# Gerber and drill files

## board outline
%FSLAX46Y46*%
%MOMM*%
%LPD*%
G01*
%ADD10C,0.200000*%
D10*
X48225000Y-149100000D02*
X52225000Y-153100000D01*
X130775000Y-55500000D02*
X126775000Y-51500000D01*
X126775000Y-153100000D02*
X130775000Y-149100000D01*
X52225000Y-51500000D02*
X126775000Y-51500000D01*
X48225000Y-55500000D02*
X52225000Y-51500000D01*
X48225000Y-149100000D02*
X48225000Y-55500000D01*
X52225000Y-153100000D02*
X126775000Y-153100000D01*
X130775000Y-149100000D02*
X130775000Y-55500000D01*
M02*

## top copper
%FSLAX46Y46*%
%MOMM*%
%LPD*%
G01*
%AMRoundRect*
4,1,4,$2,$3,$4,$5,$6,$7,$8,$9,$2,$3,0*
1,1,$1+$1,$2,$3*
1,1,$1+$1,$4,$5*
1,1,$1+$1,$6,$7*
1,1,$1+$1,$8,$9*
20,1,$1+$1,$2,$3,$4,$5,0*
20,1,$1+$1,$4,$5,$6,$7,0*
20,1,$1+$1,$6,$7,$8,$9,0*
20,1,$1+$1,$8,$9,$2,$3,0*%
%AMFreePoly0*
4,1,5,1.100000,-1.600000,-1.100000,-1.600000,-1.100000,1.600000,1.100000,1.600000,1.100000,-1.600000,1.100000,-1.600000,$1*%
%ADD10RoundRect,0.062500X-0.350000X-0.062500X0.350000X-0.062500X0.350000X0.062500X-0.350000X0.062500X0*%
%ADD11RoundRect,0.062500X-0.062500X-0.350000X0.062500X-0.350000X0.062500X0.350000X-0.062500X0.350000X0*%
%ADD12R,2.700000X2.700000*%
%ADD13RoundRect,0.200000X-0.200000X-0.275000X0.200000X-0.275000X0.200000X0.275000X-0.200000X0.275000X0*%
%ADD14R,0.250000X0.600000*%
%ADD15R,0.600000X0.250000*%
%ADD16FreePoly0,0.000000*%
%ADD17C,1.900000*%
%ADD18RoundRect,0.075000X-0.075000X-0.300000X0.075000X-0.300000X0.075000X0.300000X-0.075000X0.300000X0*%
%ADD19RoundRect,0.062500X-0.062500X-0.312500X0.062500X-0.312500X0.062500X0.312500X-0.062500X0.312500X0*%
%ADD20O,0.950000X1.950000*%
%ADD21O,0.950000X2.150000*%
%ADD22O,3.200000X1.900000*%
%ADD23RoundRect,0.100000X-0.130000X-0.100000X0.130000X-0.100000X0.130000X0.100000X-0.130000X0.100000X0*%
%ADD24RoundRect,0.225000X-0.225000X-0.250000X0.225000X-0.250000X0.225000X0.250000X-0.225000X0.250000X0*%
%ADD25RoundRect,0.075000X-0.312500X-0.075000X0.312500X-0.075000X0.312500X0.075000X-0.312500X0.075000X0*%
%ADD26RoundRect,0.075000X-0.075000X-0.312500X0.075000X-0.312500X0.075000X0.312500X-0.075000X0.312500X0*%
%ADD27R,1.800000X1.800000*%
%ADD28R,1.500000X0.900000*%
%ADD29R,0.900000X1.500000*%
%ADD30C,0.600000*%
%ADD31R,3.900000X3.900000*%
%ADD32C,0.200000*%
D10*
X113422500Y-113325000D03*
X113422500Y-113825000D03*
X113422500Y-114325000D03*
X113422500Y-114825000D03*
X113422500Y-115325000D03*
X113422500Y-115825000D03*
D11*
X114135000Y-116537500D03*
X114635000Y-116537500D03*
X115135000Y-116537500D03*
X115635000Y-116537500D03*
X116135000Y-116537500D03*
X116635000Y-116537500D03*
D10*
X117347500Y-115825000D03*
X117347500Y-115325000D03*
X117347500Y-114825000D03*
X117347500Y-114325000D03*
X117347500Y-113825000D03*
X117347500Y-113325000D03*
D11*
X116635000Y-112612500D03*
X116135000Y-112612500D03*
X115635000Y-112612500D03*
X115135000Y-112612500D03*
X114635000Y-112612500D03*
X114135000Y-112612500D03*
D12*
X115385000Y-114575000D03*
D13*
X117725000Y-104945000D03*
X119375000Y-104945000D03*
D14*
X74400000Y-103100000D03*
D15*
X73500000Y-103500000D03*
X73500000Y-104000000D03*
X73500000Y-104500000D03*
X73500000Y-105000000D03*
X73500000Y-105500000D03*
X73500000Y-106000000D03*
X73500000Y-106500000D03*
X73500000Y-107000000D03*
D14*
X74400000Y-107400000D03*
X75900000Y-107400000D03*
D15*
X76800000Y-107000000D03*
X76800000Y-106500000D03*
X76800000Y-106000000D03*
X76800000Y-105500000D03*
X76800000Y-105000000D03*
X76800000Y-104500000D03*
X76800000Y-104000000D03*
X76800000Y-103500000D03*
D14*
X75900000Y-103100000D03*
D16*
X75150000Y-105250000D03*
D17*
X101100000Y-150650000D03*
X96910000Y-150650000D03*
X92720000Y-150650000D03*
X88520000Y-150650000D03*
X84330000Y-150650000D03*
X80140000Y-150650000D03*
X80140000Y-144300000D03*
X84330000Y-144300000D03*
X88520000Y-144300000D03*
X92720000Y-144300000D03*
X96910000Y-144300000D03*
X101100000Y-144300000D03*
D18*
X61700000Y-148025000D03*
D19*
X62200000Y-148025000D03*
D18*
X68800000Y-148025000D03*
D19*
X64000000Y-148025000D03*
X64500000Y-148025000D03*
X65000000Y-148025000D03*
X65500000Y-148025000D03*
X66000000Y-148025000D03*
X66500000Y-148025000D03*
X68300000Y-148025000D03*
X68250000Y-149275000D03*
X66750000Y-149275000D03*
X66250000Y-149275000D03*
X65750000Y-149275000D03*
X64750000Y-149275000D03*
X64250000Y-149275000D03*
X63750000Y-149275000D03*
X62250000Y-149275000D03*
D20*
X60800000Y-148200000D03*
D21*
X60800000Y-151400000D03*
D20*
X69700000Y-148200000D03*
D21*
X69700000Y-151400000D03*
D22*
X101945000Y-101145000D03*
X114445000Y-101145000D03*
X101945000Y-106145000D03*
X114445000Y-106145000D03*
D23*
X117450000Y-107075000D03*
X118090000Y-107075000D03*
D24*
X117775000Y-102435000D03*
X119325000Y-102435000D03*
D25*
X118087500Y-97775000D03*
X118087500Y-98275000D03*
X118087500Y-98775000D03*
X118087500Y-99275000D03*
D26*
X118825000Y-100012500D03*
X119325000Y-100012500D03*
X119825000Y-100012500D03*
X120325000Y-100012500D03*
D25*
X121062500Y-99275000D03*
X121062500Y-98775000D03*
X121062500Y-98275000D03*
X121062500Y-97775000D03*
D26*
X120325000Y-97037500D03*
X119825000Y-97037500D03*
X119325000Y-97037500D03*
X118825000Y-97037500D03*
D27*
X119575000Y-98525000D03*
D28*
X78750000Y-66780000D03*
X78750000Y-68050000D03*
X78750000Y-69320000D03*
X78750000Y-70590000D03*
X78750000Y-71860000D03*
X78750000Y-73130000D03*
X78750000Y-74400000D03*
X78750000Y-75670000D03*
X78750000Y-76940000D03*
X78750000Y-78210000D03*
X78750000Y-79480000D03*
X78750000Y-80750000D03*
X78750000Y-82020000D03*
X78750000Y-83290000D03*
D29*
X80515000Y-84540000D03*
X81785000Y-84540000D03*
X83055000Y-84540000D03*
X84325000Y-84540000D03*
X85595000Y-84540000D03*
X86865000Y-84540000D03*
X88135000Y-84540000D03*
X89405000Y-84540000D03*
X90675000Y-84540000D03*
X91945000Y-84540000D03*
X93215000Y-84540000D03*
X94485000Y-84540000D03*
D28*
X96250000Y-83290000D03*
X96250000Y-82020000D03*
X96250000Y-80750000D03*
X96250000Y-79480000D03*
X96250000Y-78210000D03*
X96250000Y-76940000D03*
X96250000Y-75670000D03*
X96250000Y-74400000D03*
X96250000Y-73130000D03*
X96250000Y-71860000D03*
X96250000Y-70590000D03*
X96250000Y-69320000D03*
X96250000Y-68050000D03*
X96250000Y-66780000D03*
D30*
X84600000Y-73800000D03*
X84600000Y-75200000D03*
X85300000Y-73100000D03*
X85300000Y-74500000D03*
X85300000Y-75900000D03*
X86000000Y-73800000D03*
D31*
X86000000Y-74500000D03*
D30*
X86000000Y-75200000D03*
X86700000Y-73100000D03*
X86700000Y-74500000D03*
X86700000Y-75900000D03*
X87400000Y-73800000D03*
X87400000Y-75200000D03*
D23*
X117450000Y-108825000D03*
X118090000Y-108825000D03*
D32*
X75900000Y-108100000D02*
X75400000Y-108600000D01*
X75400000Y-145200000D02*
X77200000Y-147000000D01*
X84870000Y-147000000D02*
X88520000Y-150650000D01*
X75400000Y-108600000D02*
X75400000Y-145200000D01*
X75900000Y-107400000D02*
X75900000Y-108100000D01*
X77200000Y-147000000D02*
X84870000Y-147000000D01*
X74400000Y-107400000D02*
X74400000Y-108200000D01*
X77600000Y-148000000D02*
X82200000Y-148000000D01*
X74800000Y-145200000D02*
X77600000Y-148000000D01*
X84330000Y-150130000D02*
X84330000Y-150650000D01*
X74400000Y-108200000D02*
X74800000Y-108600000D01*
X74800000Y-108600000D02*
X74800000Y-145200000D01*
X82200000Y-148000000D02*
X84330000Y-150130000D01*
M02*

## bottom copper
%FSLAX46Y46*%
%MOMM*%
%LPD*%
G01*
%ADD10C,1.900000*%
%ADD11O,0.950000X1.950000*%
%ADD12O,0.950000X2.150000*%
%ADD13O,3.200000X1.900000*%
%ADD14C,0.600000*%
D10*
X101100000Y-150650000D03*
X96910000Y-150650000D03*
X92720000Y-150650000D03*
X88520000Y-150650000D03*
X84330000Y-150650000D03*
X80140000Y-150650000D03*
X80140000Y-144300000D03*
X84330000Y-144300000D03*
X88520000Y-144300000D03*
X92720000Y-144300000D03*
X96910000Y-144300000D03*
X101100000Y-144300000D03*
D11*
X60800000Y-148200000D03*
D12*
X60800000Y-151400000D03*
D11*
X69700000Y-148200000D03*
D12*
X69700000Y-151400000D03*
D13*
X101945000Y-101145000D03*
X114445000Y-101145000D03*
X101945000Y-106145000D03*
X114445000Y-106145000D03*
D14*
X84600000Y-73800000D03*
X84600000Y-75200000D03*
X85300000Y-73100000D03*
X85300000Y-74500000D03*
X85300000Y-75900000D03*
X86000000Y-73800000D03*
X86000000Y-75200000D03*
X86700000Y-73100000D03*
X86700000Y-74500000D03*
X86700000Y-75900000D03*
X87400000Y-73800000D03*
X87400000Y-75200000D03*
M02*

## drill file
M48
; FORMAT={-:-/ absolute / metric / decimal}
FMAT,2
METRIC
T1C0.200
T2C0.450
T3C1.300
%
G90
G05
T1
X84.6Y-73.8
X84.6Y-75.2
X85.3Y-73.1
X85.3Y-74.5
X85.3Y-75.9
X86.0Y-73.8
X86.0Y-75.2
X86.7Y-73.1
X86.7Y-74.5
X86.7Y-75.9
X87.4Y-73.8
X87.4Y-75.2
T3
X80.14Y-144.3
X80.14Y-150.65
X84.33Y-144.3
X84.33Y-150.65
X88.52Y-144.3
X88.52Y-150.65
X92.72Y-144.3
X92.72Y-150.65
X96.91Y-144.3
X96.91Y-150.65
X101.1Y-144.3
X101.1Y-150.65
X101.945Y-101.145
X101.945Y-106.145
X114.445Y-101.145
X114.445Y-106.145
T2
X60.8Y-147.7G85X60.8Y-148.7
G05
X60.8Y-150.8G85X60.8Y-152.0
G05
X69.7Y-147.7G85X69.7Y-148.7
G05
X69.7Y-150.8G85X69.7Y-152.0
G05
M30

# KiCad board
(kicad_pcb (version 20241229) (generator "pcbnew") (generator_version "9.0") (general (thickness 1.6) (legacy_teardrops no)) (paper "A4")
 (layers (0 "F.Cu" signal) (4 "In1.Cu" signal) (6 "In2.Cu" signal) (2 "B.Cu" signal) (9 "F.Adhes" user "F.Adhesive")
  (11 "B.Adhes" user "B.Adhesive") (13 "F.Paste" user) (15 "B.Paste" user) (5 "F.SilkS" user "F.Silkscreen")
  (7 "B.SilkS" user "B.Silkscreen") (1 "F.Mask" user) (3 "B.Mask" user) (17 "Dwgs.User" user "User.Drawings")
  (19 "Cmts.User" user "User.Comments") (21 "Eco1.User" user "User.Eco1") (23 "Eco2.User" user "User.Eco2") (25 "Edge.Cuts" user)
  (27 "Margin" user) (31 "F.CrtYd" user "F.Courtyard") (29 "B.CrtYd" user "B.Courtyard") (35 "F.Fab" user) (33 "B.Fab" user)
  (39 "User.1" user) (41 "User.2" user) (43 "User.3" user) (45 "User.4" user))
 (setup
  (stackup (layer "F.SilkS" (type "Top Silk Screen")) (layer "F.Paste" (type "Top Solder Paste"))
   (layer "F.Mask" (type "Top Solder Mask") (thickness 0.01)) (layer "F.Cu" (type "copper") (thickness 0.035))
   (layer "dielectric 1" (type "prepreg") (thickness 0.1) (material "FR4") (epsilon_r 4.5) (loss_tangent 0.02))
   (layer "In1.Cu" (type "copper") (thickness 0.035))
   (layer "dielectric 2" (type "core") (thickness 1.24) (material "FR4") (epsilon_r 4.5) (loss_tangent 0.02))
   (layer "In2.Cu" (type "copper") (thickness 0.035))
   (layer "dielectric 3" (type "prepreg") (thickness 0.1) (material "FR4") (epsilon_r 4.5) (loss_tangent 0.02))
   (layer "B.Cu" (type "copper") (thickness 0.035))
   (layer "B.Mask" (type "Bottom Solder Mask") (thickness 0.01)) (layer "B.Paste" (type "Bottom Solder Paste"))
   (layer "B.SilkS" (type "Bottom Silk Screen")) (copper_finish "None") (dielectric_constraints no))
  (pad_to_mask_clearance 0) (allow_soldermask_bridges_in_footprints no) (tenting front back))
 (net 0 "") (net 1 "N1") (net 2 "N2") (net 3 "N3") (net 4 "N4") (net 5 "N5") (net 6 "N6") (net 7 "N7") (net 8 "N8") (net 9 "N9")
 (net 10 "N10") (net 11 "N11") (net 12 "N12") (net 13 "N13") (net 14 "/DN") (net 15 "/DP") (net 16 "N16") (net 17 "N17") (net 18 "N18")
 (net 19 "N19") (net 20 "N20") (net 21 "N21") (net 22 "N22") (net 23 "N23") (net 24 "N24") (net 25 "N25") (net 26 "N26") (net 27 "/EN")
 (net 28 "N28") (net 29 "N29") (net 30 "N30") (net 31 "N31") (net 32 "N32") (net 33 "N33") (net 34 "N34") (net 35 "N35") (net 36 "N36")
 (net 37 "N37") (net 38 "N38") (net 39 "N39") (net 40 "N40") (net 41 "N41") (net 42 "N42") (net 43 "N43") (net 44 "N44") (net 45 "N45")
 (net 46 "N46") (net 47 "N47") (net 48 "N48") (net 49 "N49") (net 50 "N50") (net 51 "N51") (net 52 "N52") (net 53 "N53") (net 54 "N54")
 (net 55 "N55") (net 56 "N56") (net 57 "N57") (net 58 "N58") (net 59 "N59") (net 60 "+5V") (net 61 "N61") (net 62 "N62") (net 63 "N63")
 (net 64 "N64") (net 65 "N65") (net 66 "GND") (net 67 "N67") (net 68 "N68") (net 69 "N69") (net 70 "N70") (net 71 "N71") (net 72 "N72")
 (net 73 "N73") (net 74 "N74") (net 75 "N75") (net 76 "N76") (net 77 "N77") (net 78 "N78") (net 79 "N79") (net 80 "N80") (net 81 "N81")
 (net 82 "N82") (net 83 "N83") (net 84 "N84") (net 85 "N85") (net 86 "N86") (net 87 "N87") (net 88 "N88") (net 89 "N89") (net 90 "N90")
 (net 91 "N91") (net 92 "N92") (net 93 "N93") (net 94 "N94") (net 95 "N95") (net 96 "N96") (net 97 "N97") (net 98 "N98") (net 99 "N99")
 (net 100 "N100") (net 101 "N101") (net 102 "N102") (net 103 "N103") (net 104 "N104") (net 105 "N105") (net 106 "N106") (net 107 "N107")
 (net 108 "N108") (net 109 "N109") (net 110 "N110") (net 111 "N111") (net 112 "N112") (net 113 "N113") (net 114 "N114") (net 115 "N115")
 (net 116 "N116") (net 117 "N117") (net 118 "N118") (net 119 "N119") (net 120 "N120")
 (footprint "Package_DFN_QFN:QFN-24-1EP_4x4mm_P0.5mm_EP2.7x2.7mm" (layer "F.Cu") (at 115.385 114.575)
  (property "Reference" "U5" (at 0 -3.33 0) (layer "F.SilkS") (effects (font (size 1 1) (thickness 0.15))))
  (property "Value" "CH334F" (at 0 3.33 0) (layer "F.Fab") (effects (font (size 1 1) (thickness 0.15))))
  (pad "" smd roundrect (at -0.675 -0.675) (size 1.09 1.09) (layers "F.Paste") (roundrect_rratio 0.229358))
  (pad "" smd roundrect (at -0.675 0.675) (size 1.09 1.09) (layers "F.Paste") (roundrect_rratio 0.229358))
  (pad "" smd roundrect (at 0.675 -0.675) (size 1.09 1.09) (layers "F.Paste") (roundrect_rratio 0.229358))
  (pad "" smd roundrect (at 0.675 0.675) (size 1.09 1.09) (layers "F.Paste") (roundrect_rratio 0.229358))
  (pad "1" smd roundrect (at -1.9625 -1.25) (size 0.825 0.25) (layers "F.Cu" "F.Mask" "F.Paste") (roundrect_rratio 0.25) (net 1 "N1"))
  (pad "2" smd roundrect (at -1.9625 -0.75) (size 0.825 0.25) (layers "F.Cu" "F.Mask" "F.Paste") (roundrect_rratio 0.25) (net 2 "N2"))
  (pad "3" smd roundrect (at -1.9625 -0.25) (size 0.825 0.25) (layers "F.Cu" "F.Mask" "F.Paste") (roundrect_rratio 0.25) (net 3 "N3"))
  (pad "4" smd roundrect (at -1.9625 0.25) (size 0.825 0.25) (layers "F.Cu" "F.Mask" "F.Paste") (roundrect_rratio 0.25) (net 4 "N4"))
  (pad "5" smd roundrect (at -1.9625 0.75) (size 0.825 0.25) (layers "F.Cu" "F.Mask" "F.Paste") (roundrect_rratio 0.25) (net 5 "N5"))
  (pad "6" smd roundrect (at -1.9625 1.25) (size 0.825 0.25) (layers "F.Cu" "F.Mask" "F.Paste") (roundrect_rratio 0.25) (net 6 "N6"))
  (pad "7" smd roundrect (at -1.25 1.9625) (size 0.25 0.825) (layers "F.Cu" "F.Mask" "F.Paste") (roundrect_rratio 0.25) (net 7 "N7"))
  (pad "8" smd roundrect (at -0.75 1.9625) (size 0.25 0.825) (layers "F.Cu" "F.Mask" "F.Paste") (roundrect_rratio 0.25) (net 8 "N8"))
  (pad "9" smd roundrect (at -0.25 1.9625) (size 0.25 0.825) (layers "F.Cu" "F.Mask" "F.Paste") (roundrect_rratio 0.25) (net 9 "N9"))
  (pad "10" smd roundrect (at 0.25 1.9625) (size 0.25 0.825) (layers "F.Cu" "F.Mask" "F.Paste") (roundrect_rratio 0.25) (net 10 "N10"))
  (pad "11" smd roundrect (at 0.75 1.9625) (size 0.25 0.825) (layers "F.Cu" "F.Mask" "F.Paste") (roundrect_rratio 0.25) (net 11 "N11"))
  (pad "12" smd roundrect (at 1.25 1.9625) (size 0.25 0.825) (layers "F.Cu" "F.Mask" "F.Paste") (roundrect_rratio 0.25) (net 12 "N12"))
  (pad "13" smd roundrect (at 1.9625 1.25) (size 0.825 0.25) (layers "F.Cu" "F.Mask" "F.Paste") (roundrect_rratio 0.25) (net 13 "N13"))
  (pad "14" smd roundrect (at 1.9625 0.75) (size 0.825 0.25) (layers "F.Cu" "F.Mask" "F.Paste") (roundrect_rratio 0.25) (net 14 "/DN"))
  (pad "15" smd roundrect (at 1.9625 0.25) (size 0.825 0.25) (layers "F.Cu" "F.Mask" "F.Paste") (roundrect_rratio 0.25) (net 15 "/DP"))
  (pad "16" smd roundrect (at 1.9625 -0.25) (size 0.825 0.25) (layers "F.Cu" "F.Mask" "F.Paste") (roundrect_rratio 0.25) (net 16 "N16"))
  (pad "17" smd roundrect (at 1.9625 -0.75) (size 0.825 0.25) (layers "F.Cu" "F.Mask" "F.Paste") (roundrect_rratio 0.25) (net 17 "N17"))
  (pad "18" smd roundrect (at 1.9625 -1.25) (size 0.825 0.25) (layers "F.Cu" "F.Mask" "F.Paste") (roundrect_rratio 0.25) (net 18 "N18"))
  (pad "19" smd roundrect (at 1.25 -1.9625) (size 0.25 0.825) (layers "F.Cu" "F.Mask" "F.Paste") (roundrect_rratio 0.25) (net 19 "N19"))
  (pad "20" smd roundrect (at 0.75 -1.9625) (size 0.25 0.825) (layers "F.Cu" "F.Mask" "F.Paste") (roundrect_rratio 0.25) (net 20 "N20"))
  (pad "21" smd roundrect (at 0.25 -1.9625) (size 0.25 0.825) (layers "F.Cu" "F.Mask" "F.Paste") (roundrect_rratio 0.25) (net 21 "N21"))
  (pad "22" smd roundrect (at -0.25 -1.9625) (size 0.25 0.825) (layers "F.Cu" "F.Mask" "F.Paste") (roundrect_rratio 0.25) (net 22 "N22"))
  (pad "23" smd roundrect (at -0.75 -1.9625) (size 0.25 0.825) (layers "F.Cu" "F.Mask" "F.Paste") (roundrect_rratio 0.25) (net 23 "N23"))
  (pad "24" smd roundrect (at -1.25 -1.9625) (size 0.25 0.825) (layers "F.Cu" "F.Mask" "F.Paste") (roundrect_rratio 0.25) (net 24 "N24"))
  (pad "25" smd rect (at 0 0) (size 2.7 2.7) (layers "F.Cu" "F.Mask") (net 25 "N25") (zone_connect 2)))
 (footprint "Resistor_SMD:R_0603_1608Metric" (layer "F.Cu") (at 118.55 104.945)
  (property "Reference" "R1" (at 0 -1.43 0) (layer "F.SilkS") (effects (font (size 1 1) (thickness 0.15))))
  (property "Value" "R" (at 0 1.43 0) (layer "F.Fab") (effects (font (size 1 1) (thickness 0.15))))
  (pad "1" smd roundrect (at -0.825 0) (size 0.8 0.95) (layers "F.Cu" "F.Mask" "F.Paste") (roundrect_rratio 0.25) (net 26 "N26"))
  (pad "2" smd roundrect (at 0.825 0) (size 0.8 0.95) (layers "F.Cu" "F.Mask" "F.Paste") (roundrect_rratio 0.25) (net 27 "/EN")))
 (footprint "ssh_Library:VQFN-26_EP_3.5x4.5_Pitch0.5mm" (layer "F.Cu") (at 75.15 105.25)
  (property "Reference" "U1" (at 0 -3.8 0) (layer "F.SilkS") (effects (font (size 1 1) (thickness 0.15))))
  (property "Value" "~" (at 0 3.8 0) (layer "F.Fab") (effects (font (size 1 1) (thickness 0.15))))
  (pad "" smd rect (at -0.825 -1.2) (size 0.000001 0.250001) (layers "F.Paste") (thermal_bridge_angle 45))
  (pad "" smd rect (at -0.825 -0.4) (size 0.000001 0.250001) (layers "F.Paste") (thermal_bridge_angle 45))
  (pad "" smd rect (at -0.825 0.4) (size 0.000001 0.250001) (layers "F.Paste") (thermal_bridge_angle 45))
  (pad "" smd rect (at -0.825 1.2) (size 0.000001 0.250001) (layers "F.Paste") (thermal_bridge_angle 45))
  (pad "" smd rect (at -0.275 -1.2) (size 0.000001 0.250001) (layers "F.Paste") (thermal_bridge_angle 45))
  (pad "" smd rect (at -0.275 -0.4) (size 0.000001 0.250001) (layers "F.Paste") (thermal_bridge_angle 45))
  (pad "" smd rect (at -0.275 0.4) (size 0.000001 0.250001) (layers "F.Paste") (thermal_bridge_angle 45))
  (pad "" smd rect (at -0.275 1.2) (size 0.000001 0.250001) (layers "F.Paste") (thermal_bridge_angle 45))
  (pad "" smd rect (at 0.275 -1.2) (size 0.000001 0.250001) (layers "F.Paste") (thermal_bridge_angle 45))
  (pad "" smd rect (at 0.275 -0.4) (size 0.000001 0.250001) (layers "F.Paste") (thermal_bridge_angle 45))
  (pad "" smd rect (at 0.275 0.4) (size 0.000001 0.250001) (layers "F.Paste") (thermal_bridge_angle 45))
  (pad "" smd rect (at 0.275 1.2) (size 0.000001 0.250001) (layers "F.Paste") (thermal_bridge_angle 45))
  (pad "" smd rect (at 0.825 -1.2) (size 0.000001 0.250001) (layers "F.Paste") (thermal_bridge_angle 45))
  (pad "" smd rect (at 0.825 -0.4) (size 0.000001 0.250001) (layers "F.Paste") (thermal_bridge_angle 45))
  (pad "" smd rect (at 0.825 0.4) (size 0.000001 0.250001) (layers "F.Paste") (thermal_bridge_angle 45))
  (pad "" smd rect (at 0.825 1.2) (size 0.000001 0.250001) (layers "F.Paste") (thermal_bridge_angle 45))
  (pad "1" smd rect (at -0.75 -2.15) (size 0.25 0.6) (layers "F.Cu" "F.Mask" "F.Paste") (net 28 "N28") (thermal_bridge_angle 45))
  (pad "2" smd rect (at -1.65 -1.75 90) (size 0.25 0.6) (layers "F.Cu" "F.Mask" "F.Paste") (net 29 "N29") (thermal_bridge_angle 45))
  (pad "3" smd rect (at -1.65 -1.25 90) (size 0.25 0.6) (layers "F.Cu" "F.Mask" "F.Paste") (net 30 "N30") (thermal_bridge_angle 45))
  (pad "4" smd rect (at -1.65 -0.75 90) (size 0.25 0.6) (layers "F.Cu" "F.Mask" "F.Paste") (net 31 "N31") (thermal_bridge_angle 45))
  (pad "5" smd rect (at -1.65 -0.25 90) (size 0.25 0.6) (layers "F.Cu" "F.Mask" "F.Paste") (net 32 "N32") (thermal_bridge_angle 45))
  (pad "6" smd rect (at -1.65 0.25 90) (size 0.25 0.6) (layers "F.Cu" "F.Mask" "F.Paste") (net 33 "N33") (thermal_bridge_angle 45))
  (pad "7" smd rect (at -1.65 0.75 90) (size 0.25 0.6) (layers "F.Cu" "F.Mask" "F.Paste") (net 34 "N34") (thermal_bridge_angle 45))
  (pad "8" smd rect (at -1.65 1.25 90) (size 0.25 0.6) (layers "F.Cu" "F.Mask" "F.Paste") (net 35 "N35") (thermal_bridge_angle 45))
  (pad "9" smd rect (at -1.65 1.75 90) (size 0.25 0.6) (layers "F.Cu" "F.Mask" "F.Paste") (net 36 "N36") (thermal_bridge_angle 45))
  (pad "10" smd rect (at -0.75 2.15) (size 0.25 0.6) (layers "F.Cu" "F.Mask" "F.Paste") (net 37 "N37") (thermal_bridge_angle 45))
  (pad "11" smd rect (at 0.75 2.15) (size 0.25 0.6) (layers "F.Cu" "F.Mask" "F.Paste") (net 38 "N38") (thermal_bridge_angle 45))
  (pad "12" smd rect (at 1.65 1.75 90) (size 0.25 0.6) (layers "F.Cu" "F.Mask" "F.Paste") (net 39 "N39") (thermal_bridge_angle 45))
  (pad "13" smd rect (at 1.65 1.25 90) (size 0.25 0.6) (layers "F.Cu" "F.Mask" "F.Paste") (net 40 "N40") (thermal_bridge_angle 45))
  (pad "14" smd rect (at 1.65 0.75 90) (size 0.25 0.6) (layers "F.Cu" "F.Mask" "F.Paste") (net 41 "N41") (thermal_bridge_angle 45))
  (pad "15" smd rect (at 1.65 0.25 90) (size 0.25 0.6) (layers "F.Cu" "F.Mask" "F.Paste") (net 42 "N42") (thermal_bridge_angle 45))
  (pad "16" smd rect (at 1.65 -0.25 90) (size 0.25 0.6) (layers "F.Cu" "F.Mask" "F.Paste") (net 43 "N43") (thermal_bridge_angle 45))
  (pad "17" smd rect (at 1.65 -0.75 90) (size 0.25 0.6) (layers "F.Cu" "F.Mask" "F.Paste") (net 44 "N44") (thermal_bridge_angle 45))
  (pad "18" smd rect (at 1.65 -1.25 90) (size 0.25 0.6) (layers "F.Cu" "F.Mask" "F.Paste") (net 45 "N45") (thermal_bridge_angle 45))
  (pad "19" smd rect (at 1.65 -1.75 90) (size 0.25 0.6) (layers "F.Cu" "F.Mask" "F.Paste") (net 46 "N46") (thermal_bridge_angle 45))
  (pad "20" smd rect (at 0.75 -2.15) (size 0.25 0.6) (layers "F.Cu" "F.Mask" "F.Paste") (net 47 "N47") (thermal_bridge_angle 45))
  (pad "21" smd custom (at 0 0) (size 2.2 3.2) (layers "F.Cu" "F.Mask") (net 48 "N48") (options (clearance outline) (anchor rect))
   (primitives)
   (teardrops (best_length_ratio 0.5) (max_length 1) (best_width_ratio 1) (max_width 2) (curved_edges no) (filter_ratio 0.9) (enabled yes)
    (allow_two_segments yes) (prefer_zone_connections yes))))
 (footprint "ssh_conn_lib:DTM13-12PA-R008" (layer "F.Cu") (at 90.62 153.1)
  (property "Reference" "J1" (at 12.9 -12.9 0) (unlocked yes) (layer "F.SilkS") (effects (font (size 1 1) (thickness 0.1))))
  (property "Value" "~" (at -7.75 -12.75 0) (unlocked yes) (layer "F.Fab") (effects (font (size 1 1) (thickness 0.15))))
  (pad "1" thru_hole circle (at 10.48 -2.45) (size 1.9 1.9) (drill 1.3) (layers "*.Cu" "*.Mask") (remove_unused_layers no) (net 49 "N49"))
  (pad "2" thru_hole circle (at 6.29 -2.45) (size 1.9 1.9) (drill 1.3) (layers "*.Cu" "*.Mask") (remove_unused_layers no) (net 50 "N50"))
  (pad "3" thru_hole circle (at 2.1 -2.45) (size 1.9 1.9) (drill 1.3) (layers "*.Cu" "*.Mask") (remove_unused_layers no) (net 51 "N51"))
  (pad "4" thru_hole circle (at -2.1 -2.45) (size 1.9 1.9) (drill 1.3) (layers "*.Cu" "*.Mask") (remove_unused_layers no) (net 38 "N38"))
  (pad "5" thru_hole circle (at -6.29 -2.45) (size 1.9 1.9) (drill 1.3) (layers "*.Cu" "*.Mask") (remove_unused_layers no) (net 37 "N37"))
  (pad "6" thru_hole circle (at -10.48 -2.45) (size 1.9 1.9) (drill 1.3) (layers "*.Cu" "*.Mask") (remove_unused_layers no) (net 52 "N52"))
  (pad "7" thru_hole circle (at -10.48 -8.8) (size 1.9 1.9) (drill 1.3) (layers "*.Cu" "*.Mask") (remove_unused_layers no) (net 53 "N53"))
  (pad "8" thru_hole circle (at -6.29 -8.8) (size 1.9 1.9) (drill 1.3) (layers "*.Cu" "*.Mask") (remove_unused_layers no) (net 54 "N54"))
  (pad "9" thru_hole circle (at -2.1 -8.8) (size 1.9 1.9) (drill 1.3) (layers "*.Cu" "*.Mask") (remove_unused_layers no) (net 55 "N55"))
  (pad "10" thru_hole circle (at 2.1 -8.8) (size 1.9 1.9) (drill 1.3) (layers "*.Cu" "*.Mask") (remove_unused_layers no) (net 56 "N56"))
  (pad "11" thru_hole circle (at 6.29 -8.8) (size 1.9 1.9) (drill 1.3) (layers "*.Cu" "*.Mask") (remove_unused_layers no) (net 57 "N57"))
  (pad "12" thru_hole circle (at 10.48 -8.8) (size 1.9 1.9) (drill 1.3) (layers "*.Cu" "*.Mask") (remove_unused_layers no) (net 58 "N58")))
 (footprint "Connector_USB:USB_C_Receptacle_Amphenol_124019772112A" (layer "F.Cu") (at 65.25 151.225)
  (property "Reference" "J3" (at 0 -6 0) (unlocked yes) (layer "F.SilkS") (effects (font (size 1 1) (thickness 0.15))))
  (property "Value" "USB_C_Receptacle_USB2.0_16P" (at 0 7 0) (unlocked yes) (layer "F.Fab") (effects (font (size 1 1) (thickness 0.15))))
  (pad "A1" smd roundrect (at -3.55 -3.2) (size 0.3 0.75) (layers "F.Cu" "F.Mask" "F.Paste") (roundrect_rratio 0.25) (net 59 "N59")
   (thermal_bridge_angle 45))
  (pad "A1" smd roundrect (at -3.05 -3.2) (size 0.25 0.75) (layers "F.Cu" "F.Mask" "F.Paste") (roundrect_rratio 0.25) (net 59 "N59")
   (thermal_bridge_angle 45))
  (pad "A1" smd roundrect (at 3.55 -3.2) (size 0.3 0.75) (layers "F.Cu" "F.Mask" "F.Paste") (roundrect_rratio 0.25) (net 59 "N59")
   (thermal_bridge_angle 45))
  (pad "A4" smd roundrect (at -1.25 -3.2) (size 0.25 0.75) (layers "F.Cu" "F.Mask" "F.Paste") (roundrect_rratio 0.25) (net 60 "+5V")
   (thermal_bridge_angle 45))
  (pad "A5" smd roundrect (at -0.75 -3.2) (size 0.25 0.75) (layers "F.Cu" "F.Mask" "F.Paste") (roundrect_rratio 0.25) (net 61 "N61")
   (thermal_bridge_angle 45))
  (pad "A6" smd roundrect (at -0.25 -3.2) (size 0.25 0.75) (layers "F.Cu" "F.Mask" "F.Paste") (roundrect_rratio 0.25) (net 15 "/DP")
   (thermal_bridge_angle 45))
  (pad "A7" smd roundrect (at 0.25 -3.2) (size 0.25 0.75) (layers "F.Cu" "F.Mask" "F.Paste") (roundrect_rratio 0.25) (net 14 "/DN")
   (thermal_bridge_angle 45))
  (pad "A8" smd roundrect (at 0.75 -3.2) (size 0.25 0.75) (layers "F.Cu" "F.Mask" "F.Paste") (roundrect_rratio 0.25) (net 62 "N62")
   (thermal_bridge_angle 45))
  (pad "A9" smd roundrect (at 1.25 -3.2) (size 0.25 0.75) (layers "F.Cu" "F.Mask" "F.Paste") (roundrect_rratio 0.25) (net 60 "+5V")
   (thermal_bridge_angle 45))
  (pad "A12" smd roundrect (at 3.05 -3.2) (size 0.25 0.75) (layers "F.Cu" "F.Mask" "F.Paste") (roundrect_rratio 0.25) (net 59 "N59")
   (thermal_bridge_angle 45))
  (pad "B1" smd roundrect (at 3 -1.95) (size 0.25 0.75) (layers "F.Cu" "F.Mask" "F.Paste") (roundrect_rratio 0.25) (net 59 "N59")
   (thermal_bridge_angle 45))
  (pad "B4" smd roundrect (at 1.5 -1.95) (size 0.25 0.75) (layers "F.Cu" "F.Mask" "F.Paste") (roundrect_rratio 0.25) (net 60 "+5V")
   (thermal_bridge_angle 45))
  (pad "B5" smd roundrect (at 1 -1.95) (size 0.25 0.75) (layers "F.Cu" "F.Mask" "F.Paste") (roundrect_rratio 0.25) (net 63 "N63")
   (thermal_bridge_angle 45))
  (pad "B6" smd roundrect (at 0.5 -1.95) (size 0.25 0.75) (layers "F.Cu" "F.Mask" "F.Paste") (roundrect_rratio 0.25) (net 15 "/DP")
   (thermal_bridge_angle 45))
  (pad "B7" smd roundrect (at -0.5 -1.95) (size 0.25 0.75) (layers "F.Cu" "F.Mask" "F.Paste") (roundrect_rratio 0.25) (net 14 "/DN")
   (thermal_bridge_angle 45))
  (pad "B8" smd roundrect (at -1 -1.95) (size 0.25 0.75) (layers "F.Cu" "F.Mask" "F.Paste") (roundrect_rratio 0.25) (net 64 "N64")
   (thermal_bridge_angle 45))
  (pad "B9" smd roundrect (at -1.5 -1.95) (size 0.25 0.75) (layers "F.Cu" "F.Mask" "F.Paste") (roundrect_rratio 0.25) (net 60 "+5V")
   (thermal_bridge_angle 45))
  (pad "B12" smd roundrect (at -3 -1.95) (size 0.25 0.75) (layers "F.Cu" "F.Mask" "F.Paste") (roundrect_rratio 0.25) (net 59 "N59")
   (thermal_bridge_angle 45))
  (pad "S1" thru_hole oval (at -4.45 -3.025) (size 0.95 1.95) (drill oval 0.45 1.45) (layers "*.Cu" "*.Mask") (remove_unused_layers no)
   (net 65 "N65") (thermal_bridge_angle 45))
  (pad "S1" thru_hole oval (at -4.45 0.175) (size 0.95 2.15) (drill oval 0.45 1.65) (layers "*.Cu" "*.Mask") (remove_unused_layers no)
   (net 65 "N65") (thermal_bridge_angle 45))
  (pad "S1" thru_hole oval (at 4.45 -3.025) (size 0.95 1.95) (drill oval 0.45 1.45) (layers "*.Cu" "*.Mask") (remove_unused_layers no)
   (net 65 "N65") (thermal_bridge_angle 45))
  (pad "S1" thru_hole oval (at 4.45 0.175) (size 0.95 2.15) (drill oval 0.45 1.65) (layers "*.Cu" "*.Mask") (remove_unused_layers no)
   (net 65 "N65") (thermal_bridge_angle 45)))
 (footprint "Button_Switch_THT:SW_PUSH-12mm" (layer "F.Cu") (at 101.945 101.145)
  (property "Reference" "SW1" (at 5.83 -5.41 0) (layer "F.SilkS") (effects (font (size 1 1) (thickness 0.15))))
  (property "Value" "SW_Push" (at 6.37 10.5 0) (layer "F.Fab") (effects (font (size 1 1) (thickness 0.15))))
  (pad "1" thru_hole oval (at 0 0) (size 3.2 1.9) (drill 1.3) (layers "*.Cu" "*.Mask") (remove_unused_layers no) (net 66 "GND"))
  (pad "1" thru_hole oval (at 12.5 0) (size 3.2 1.9) (drill 1.3) (layers "*.Cu" "*.Mask") (remove_unused_layers no) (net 66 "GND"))
  (pad "2" thru_hole oval (at 0 5) (size 3.2 1.9) (drill 1.3) (layers "*.Cu" "*.Mask") (remove_unused_layers no) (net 26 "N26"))
  (pad "2" thru_hole oval (at 12.5 5) (size 3.2 1.9) (drill 1.3) (layers "*.Cu" "*.Mask") (remove_unused_layers no) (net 26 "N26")))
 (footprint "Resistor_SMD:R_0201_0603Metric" (layer "F.Cu") (at 117.77 107.075)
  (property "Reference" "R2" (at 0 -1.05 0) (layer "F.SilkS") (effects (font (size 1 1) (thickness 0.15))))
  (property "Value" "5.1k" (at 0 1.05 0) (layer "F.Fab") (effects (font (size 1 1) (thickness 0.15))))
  (pad "" smd roundrect (at -0.345 0) (size 0.318 0.36) (layers "F.Paste") (roundrect_rratio 0.25))
  (pad "" smd roundrect (at 0.345 0) (size 0.318 0.36) (layers "F.Paste") (roundrect_rratio 0.25))
  (pad "1" smd roundrect (at -0.32 0) (size 0.46 0.4) (layers "F.Cu" "F.Mask") (roundrect_rratio 0.25) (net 61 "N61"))
  (pad "2" smd roundrect (at 0.32 0) (size 0.46 0.4) (layers "F.Cu" "F.Mask") (roundrect_rratio 0.25) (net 66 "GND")))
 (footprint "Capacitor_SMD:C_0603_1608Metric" (layer "F.Cu") (at 118.55 102.435)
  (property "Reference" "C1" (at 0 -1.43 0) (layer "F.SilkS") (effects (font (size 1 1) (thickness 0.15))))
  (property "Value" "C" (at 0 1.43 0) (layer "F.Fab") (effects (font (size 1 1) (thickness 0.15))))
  (pad "1" smd roundrect (at -0.775 0) (size 0.9 0.95) (layers "F.Cu" "F.Mask" "F.Paste") (roundrect_rratio 0.25) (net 26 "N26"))
  (pad "2" smd roundrect (at 0.775 0) (size 0.9 0.95) (layers "F.Cu" "F.Mask" "F.Paste") (roundrect_rratio 0.25) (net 66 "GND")))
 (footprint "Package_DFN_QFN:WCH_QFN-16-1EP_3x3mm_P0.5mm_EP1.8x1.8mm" (layer "F.Cu") (at 119.575 98.525)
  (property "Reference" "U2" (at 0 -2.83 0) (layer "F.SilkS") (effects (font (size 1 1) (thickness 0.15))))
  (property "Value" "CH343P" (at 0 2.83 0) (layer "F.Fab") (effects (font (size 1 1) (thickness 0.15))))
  (pad "" smd roundrect (at -0.45 -0.45) (size 0.73 0.73) (layers "F.Paste") (roundrect_rratio 0.25))
  (pad "" smd roundrect (at -0.45 0.45) (size 0.73 0.73) (layers "F.Paste") (roundrect_rratio 0.25))
  (pad "" smd roundrect (at 0.45 -0.45) (size 0.73 0.73) (layers "F.Paste") (roundrect_rratio 0.25))
  (pad "" smd roundrect (at 0.45 0.45) (size 0.73 0.73) (layers "F.Paste") (roundrect_rratio 0.25))
  (pad "1" smd roundrect (at -1.4875 -0.75) (size 0.775 0.3) (layers "F.Cu" "F.Mask" "F.Paste") (roundrect_rratio 0.25) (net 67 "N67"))
  (pad "2" smd roundrect (at -1.4875 -0.25) (size 0.775 0.3) (layers "F.Cu" "F.Mask" "F.Paste") (roundrect_rratio 0.25) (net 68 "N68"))
  (pad "3" smd roundrect (at -1.4875 0.25) (size 0.775 0.3) (layers "F.Cu" "F.Mask" "F.Paste") (roundrect_rratio 0.25) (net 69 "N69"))
  (pad "4" smd roundrect (at -1.4875 0.75) (size 0.775 0.3) (layers "F.Cu" "F.Mask" "F.Paste") (roundrect_rratio 0.25) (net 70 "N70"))
  (pad "5" smd roundrect (at -0.75 1.4875) (size 0.3 0.775) (layers "F.Cu" "F.Mask" "F.Paste") (roundrect_rratio 0.25) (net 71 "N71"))
  (pad "6" smd roundrect (at -0.25 1.4875) (size 0.3 0.775) (layers "F.Cu" "F.Mask" "F.Paste") (roundrect_rratio 0.25) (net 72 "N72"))
  (pad "7" smd roundrect (at 0.25 1.4875) (size 0.3 0.775) (layers "F.Cu" "F.Mask" "F.Paste") (roundrect_rratio 0.25) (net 10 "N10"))
  (pad "8" smd roundrect (at 0.75 1.4875) (size 0.3 0.775) (layers "F.Cu" "F.Mask" "F.Paste") (roundrect_rratio 0.25) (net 9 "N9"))
  (pad "9" smd roundrect (at 1.4875 0.75) (size 0.775 0.3) (layers "F.Cu" "F.Mask" "F.Paste") (roundrect_rratio 0.25) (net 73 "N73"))
  (pad "10" smd roundrect (at 1.4875 0.25) (size 0.775 0.3) (layers "F.Cu" "F.Mask" "F.Paste") (roundrect_rratio 0.25) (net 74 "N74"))
  (pad "11" smd roundrect (at 1.4875 -0.25) (size 0.775 0.3) (layers "F.Cu" "F.Mask" "F.Paste") (roundrect_rratio 0.25) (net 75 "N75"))
  (pad "12" smd roundrect (at 1.4875 -0.75) (size 0.775 0.3) (layers "F.Cu" "F.Mask" "F.Paste") (roundrect_rratio 0.25) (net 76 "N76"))
  (pad "13" smd roundrect (at 0.75 -1.4875) (size 0.3 0.775) (layers "F.Cu" "F.Mask" "F.Paste") (roundrect_rratio 0.25) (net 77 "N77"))
  (pad "14" smd roundrect (at 0.25 -1.4875) (size 0.3 0.775) (layers "F.Cu" "F.Mask" "F.Paste") (roundrect_rratio 0.25) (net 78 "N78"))
  (pad "15" smd roundrect (at -0.25 -1.4875) (size 0.3 0.775) (layers "F.Cu" "F.Mask" "F.Paste") (roundrect_rratio 0.25) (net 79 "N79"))
  (pad "16" smd roundrect (at -0.75 -1.4875) (size 0.3 0.775) (layers "F.Cu" "F.Mask" "F.Paste") (roundrect_rratio 0.25) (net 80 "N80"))
  (pad "17" smd rect (at 0 0) (size 1.8 1.8) (layers "F.Cu" "F.Mask") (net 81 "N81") (zone_connect 2)))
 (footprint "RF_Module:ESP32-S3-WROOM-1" (layer "F.Cu") (at 87.5 72.04)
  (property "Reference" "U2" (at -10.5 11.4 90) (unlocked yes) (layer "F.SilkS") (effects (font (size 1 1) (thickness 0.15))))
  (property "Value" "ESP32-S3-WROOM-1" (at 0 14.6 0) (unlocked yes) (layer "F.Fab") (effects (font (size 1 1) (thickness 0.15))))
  (pad "" smd rect (at -2.9 1.06) (size 0.9 0.9) (layers "F.Paste"))
  (pad "" smd rect (at -2.9 2.46 270) (size 0.9 0.9) (layers "F.Paste"))
  (pad "" smd rect (at -2.9 3.86) (size 0.9 0.9) (layers "F.Paste"))
  (pad "" smd rect (at -1.5 1.06 270) (size 0.9 0.9) (layers "F.Paste"))
  (pad "" smd rect (at -1.5 2.46 270) (size 0.9 0.9) (layers "F.Paste"))
  (pad "" smd rect (at -1.5 3.86 270) (size 0.9 0.9) (layers "F.Paste"))
  (pad "" smd rect (at -0.1 1.06 270) (size 0.9 0.9) (layers "F.Paste"))
  (pad "" smd rect (at -0.1 2.46 270) (size 0.9 0.9) (layers "F.Paste"))
  (pad "" smd rect (at -0.1 3.86 270) (size 0.9 0.9) (layers "F.Paste"))
  (pad "1" smd rect (at -8.75 -5.26) (size 1.5 0.9) (layers "F.Cu" "F.Mask" "F.Paste") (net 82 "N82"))
  (pad "2" smd rect (at -8.75 -3.99) (size 1.5 0.9) (layers "F.Cu" "F.Mask" "F.Paste") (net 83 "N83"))
  (pad "3" smd rect (at -8.75 -2.72) (size 1.5 0.9) (layers "F.Cu" "F.Mask" "F.Paste") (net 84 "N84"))
  (pad "4" smd rect (at -8.75 -1.45) (size 1.5 0.9) (layers "F.Cu" "F.Mask" "F.Paste") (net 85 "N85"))
  (pad "5" smd rect (at -8.75 -0.18) (size 1.5 0.9) (layers "F.Cu" "F.Mask" "F.Paste") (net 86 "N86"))
  (pad "6" smd rect (at -8.75 1.09) (size 1.5 0.9) (layers "F.Cu" "F.Mask" "F.Paste") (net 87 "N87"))
  (pad "7" smd rect (at -8.75 2.36) (size 1.5 0.9) (layers "F.Cu" "F.Mask" "F.Paste") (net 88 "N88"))
  (pad "8" smd rect (at -8.75 3.63) (size 1.5 0.9) (layers "F.Cu" "F.Mask" "F.Paste") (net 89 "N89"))
  (pad "9" smd rect (at -8.75 4.9) (size 1.5 0.9) (layers "F.Cu" "F.Mask" "F.Paste") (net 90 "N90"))
  (pad "10" smd rect (at -8.75 6.17) (size 1.5 0.9) (layers "F.Cu" "F.Mask" "F.Paste") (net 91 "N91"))
  (pad "11" smd rect (at -8.75 7.44) (size 1.5 0.9) (layers "F.Cu" "F.Mask" "F.Paste") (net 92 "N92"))
  (pad "12" smd rect (at -8.75 8.71) (size 1.5 0.9) (layers "F.Cu" "F.Mask" "F.Paste") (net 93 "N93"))
  (pad "13" smd rect (at -8.75 9.98) (size 1.5 0.9) (layers "F.Cu" "F.Mask" "F.Paste") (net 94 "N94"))
  (pad "14" smd rect (at -8.75 11.25 180) (size 1.5 0.9) (layers "F.Cu" "F.Mask" "F.Paste") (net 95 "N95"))
  (pad "15" smd rect (at -6.985 12.5 270) (size 1.5 0.9) (layers "F.Cu" "F.Mask" "F.Paste") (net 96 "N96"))
  (pad "16" smd rect (at -5.715 12.5 270) (size 1.5 0.9) (layers "F.Cu" "F.Mask" "F.Paste") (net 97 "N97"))
  (pad "17" smd rect (at -4.445 12.5 270) (size 1.5 0.9) (layers "F.Cu" "F.Mask" "F.Paste") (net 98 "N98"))
  (pad "18" smd rect (at -3.175 12.5 270) (size 1.5 0.9) (layers "F.Cu" "F.Mask" "F.Paste") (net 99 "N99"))
  (pad "19" smd rect (at -1.905 12.5 270) (size 1.5 0.9) (layers "F.Cu" "F.Mask" "F.Paste") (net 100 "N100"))
  (pad "20" smd rect (at -0.635 12.5 270) (size 1.5 0.9) (layers "F.Cu" "F.Mask" "F.Paste") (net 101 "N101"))
  (pad "21" smd rect (at 0.635 12.5 270) (size 1.5 0.9) (layers "F.Cu" "F.Mask" "F.Paste") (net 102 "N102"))
  (pad "22" smd rect (at 1.905 12.5 270) (size 1.5 0.9) (layers "F.Cu" "F.Mask" "F.Paste") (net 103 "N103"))
  (pad "23" smd rect (at 3.175 12.5 270) (size 1.5 0.9) (layers "F.Cu" "F.Mask" "F.Paste") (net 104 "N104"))
  (pad "24" smd rect (at 4.445 12.5 270) (size 1.5 0.9) (layers "F.Cu" "F.Mask" "F.Paste") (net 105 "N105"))
  (pad "25" smd rect (at 5.715 12.5 270) (size 1.5 0.9) (layers "F.Cu" "F.Mask" "F.Paste") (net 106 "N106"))
  (pad "26" smd rect (at 6.985 12.5 270) (size 1.5 0.9) (layers "F.Cu" "F.Mask" "F.Paste") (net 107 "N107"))
  (pad "27" smd rect (at 8.75 11.25) (size 1.5 0.9) (layers "F.Cu" "F.Mask" "F.Paste") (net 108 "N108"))
  (pad "28" smd rect (at 8.75 9.98) (size 1.5 0.9) (layers "F.Cu" "F.Mask" "F.Paste") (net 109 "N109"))
  (pad "29" smd rect (at 8.75 8.71) (size 1.5 0.9) (layers "F.Cu" "F.Mask" "F.Paste") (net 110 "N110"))
  (pad "30" smd rect (at 8.75 7.44) (size 1.5 0.9) (layers "F.Cu" "F.Mask" "F.Paste") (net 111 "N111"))
  (pad "31" smd rect (at 8.75 6.17) (size 1.5 0.9) (layers "F.Cu" "F.Mask" "F.Paste") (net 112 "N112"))
  (pad "32" smd rect (at 8.75 4.9) (size 1.5 0.9) (layers "F.Cu" "F.Mask" "F.Paste") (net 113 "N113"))
  (pad "33" smd rect (at 8.75 3.63) (size 1.5 0.9) (layers "F.Cu" "F.Mask" "F.Paste") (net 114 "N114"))
  (pad "34" smd rect (at 8.75 2.36) (size 1.5 0.9) (layers "F.Cu" "F.Mask" "F.Paste") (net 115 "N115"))
  (pad "35" smd rect (at 8.75 1.09) (size 1.5 0.9) (layers "F.Cu" "F.Mask" "F.Paste") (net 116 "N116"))
  (pad "36" smd rect (at 8.75 -0.18) (size 1.5 0.9) (layers "F.Cu" "F.Mask" "F.Paste") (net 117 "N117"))
  (pad "37" smd rect (at 8.75 -1.45) (size 1.5 0.9) (layers "F.Cu" "F.Mask" "F.Paste") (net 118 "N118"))
  (pad "38" smd rect (at 8.75 -2.72) (size 1.5 0.9) (layers "F.Cu" "F.Mask" "F.Paste") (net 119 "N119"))
  (pad "39" smd rect (at 8.75 -3.99) (size 1.5 0.9) (layers "F.Cu" "F.Mask" "F.Paste") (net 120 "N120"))
  (pad "40" smd rect (at 8.75 -5.26) (size 1.5 0.9) (layers "F.Cu" "F.Mask" "F.Paste") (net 82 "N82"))
  (pad "41" thru_hole circle (at -2.9 1.76 90) (size 0.6 0.6) (drill 0.2) (layers "*.Cu" "F.Mask") (remove_unused_layers no) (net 82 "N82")
   (zone_connect 2))
  (pad "41" thru_hole circle (at -2.9 3.16) (size 0.6 0.6) (drill 0.2) (layers "*.Cu" "F.Mask") (remove_unused_layers no) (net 82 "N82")
   (zone_connect 2))
  (pad "41" thru_hole circle (at -2.2 1.06) (size 0.6 0.6) (drill 0.2) (layers "*.Cu" "F.Mask") (remove_unused_layers no) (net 82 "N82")
   (zone_connect 2))
  (pad "41" thru_hole circle (at -2.2 2.46) (size 0.6 0.6) (drill 0.2) (layers "*.Cu" "F.Mask") (remove_unused_layers no) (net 82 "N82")
   (zone_connect 2))
  (pad "41" thru_hole circle (at -2.2 3.86) (size 0.6 0.6) (drill 0.2) (layers "*.Cu" "F.Mask") (remove_unused_layers no) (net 82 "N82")
   (zone_connect 2))
  (pad "41" thru_hole circle (at -1.5 1.76) (size 0.6 0.6) (drill 0.2) (layers "*.Cu" "F.Mask") (remove_unused_layers no) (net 82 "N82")
   (zone_connect 2))
  (pad "41" smd rect (at -1.5 2.46 270) (size 3.9 3.9) (layers "F.Cu" "F.Mask") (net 82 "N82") (zone_connect 2))
  (pad "41" thru_hole circle (at -1.5 3.16) (size 0.6 0.6) (drill 0.2) (layers "*.Cu" "F.Mask") (remove_unused_layers no) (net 82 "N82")
   (zone_connect 2))
  (pad "41" thru_hole circle (at -0.8 1.06) (size 0.6 0.6) (drill 0.2) (layers "*.Cu" "F.Mask") (remove_unused_layers no) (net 82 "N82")
   (zone_connect 2))
  (pad "41" thru_hole circle (at -0.8 2.46) (size 0.6 0.6) (drill 0.2) (layers "*.Cu" "F.Mask") (remove_unused_layers no) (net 82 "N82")
   (zone_connect 2))
  (pad "41" thru_hole circle (at -0.8 3.86) (size 0.6 0.6) (drill 0.2) (layers "*.Cu" "F.Mask") (remove_unused_layers no) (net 82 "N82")
   (zone_connect 2))
  (pad "41" thru_hole circle (at -0.1 1.76) (size 0.6 0.6) (drill 0.2) (layers "*.Cu" "F.Mask") (remove_unused_layers no) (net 82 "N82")
   (zone_connect 2))
  (pad "41" thru_hole circle (at -0.1 3.16) (size 0.6 0.6) (drill 0.2) (layers "*.Cu" "F.Mask") (remove_unused_layers no) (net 82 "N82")
   (zone_connect 2))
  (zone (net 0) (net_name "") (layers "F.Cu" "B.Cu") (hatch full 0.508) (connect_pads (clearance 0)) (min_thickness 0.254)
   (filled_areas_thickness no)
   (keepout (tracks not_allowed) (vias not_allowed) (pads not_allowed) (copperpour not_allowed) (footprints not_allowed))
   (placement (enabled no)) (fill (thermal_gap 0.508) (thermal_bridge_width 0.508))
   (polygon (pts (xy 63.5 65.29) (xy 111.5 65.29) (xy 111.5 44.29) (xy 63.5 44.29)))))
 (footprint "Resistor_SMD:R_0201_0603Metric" (layer "F.Cu") (at 117.77 108.825)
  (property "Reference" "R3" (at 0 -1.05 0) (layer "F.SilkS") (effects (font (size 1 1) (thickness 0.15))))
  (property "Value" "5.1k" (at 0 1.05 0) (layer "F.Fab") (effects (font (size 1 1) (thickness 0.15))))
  (pad "" smd roundrect (at -0.345 0) (size 0.318 0.36) (layers "F.Paste") (roundrect_rratio 0.25))
  (pad "" smd roundrect (at 0.345 0) (size 0.318 0.36) (layers "F.Paste") (roundrect_rratio 0.25))
  (pad "1" smd roundrect (at -0.32 0) (size 0.46 0.4) (layers "F.Cu" "F.Mask") (roundrect_rratio 0.25) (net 63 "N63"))
  (pad "2" smd roundrect (at 0.32 0) (size 0.46 0.4) (layers "F.Cu" "F.Mask") (roundrect_rratio 0.25) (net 66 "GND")))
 (gr_line (start 48.225 149.1) (end 52.225 153.1) (stroke (width 0.2) (type default)) (layer "Edge.Cuts"))
 (gr_line (start 130.775 55.5) (end 126.775 51.5) (stroke (width 0.2) (type default)) (layer "Edge.Cuts"))
 (gr_line (start 126.775 153.1) (end 130.775 149.1) (stroke (width 0.2) (type default)) (layer "Edge.Cuts"))
 (gr_line (start 52.225 51.5) (end 126.775 51.5) (stroke (width 0.2) (type default)) (layer "Edge.Cuts"))
 (gr_line (start 48.225 55.5) (end 52.225 51.5) (stroke (width 0.2) (type default)) (layer "Edge.Cuts"))
 (gr_line (start 48.225 149.1) (end 48.225 55.5) (stroke (width 0.2) (type default)) (layer "Edge.Cuts"))
 (gr_line (start 52.225 153.1) (end 126.775 153.1) (stroke (width 0.2) (type default)) (layer "Edge.Cuts"))
 (gr_line (start 130.775 149.1) (end 130.775 55.5) (stroke (width 0.2) (type default)) (layer "Edge.Cuts"))
 (segment (start 75.9 108.1) (end 75.4 108.6) (width 0.2) (layer "F.Cu") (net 38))
 (segment (start 75.4 145.2) (end 77.2 147) (width 0.2) (layer "F.Cu") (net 38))
 (segment (start 84.87 147) (end 88.52 150.65) (width 0.2) (layer "F.Cu") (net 38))
 (segment (start 75.4 108.6) (end 75.4 145.2) (width 0.2) (layer "F.Cu") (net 38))
 (segment (start 75.9 107.4) (end 75.9 108.1) (width 0.2) (layer "F.Cu") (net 38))
 (segment (start 77.2 147) (end 84.87 147) (width 0.2) (layer "F.Cu") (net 38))
 (segment (start 74.4 107.4) (end 74.4 108.2) (width 0.2) (layer "F.Cu") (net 37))
 (segment (start 77.6 148) (end 82.2 148) (width 0.2) (layer "F.Cu") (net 37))
 (segment (start 74.8 145.2) (end 77.6 148) (width 0.2) (layer "F.Cu") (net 37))
 (segment (start 84.33 150.13) (end 84.33 150.65) (width 0.2) (layer "F.Cu") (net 37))
 (segment (start 74.4 108.2) (end 74.8 108.6) (width 0.2) (layer "F.Cu") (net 37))
 (segment (start 74.8 108.6) (end 74.8 145.2) (width 0.2) (layer "F.Cu") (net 37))
 (segment (start 82.2 148) (end 84.33 150.13) (width 0.2) (layer "F.Cu") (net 37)))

